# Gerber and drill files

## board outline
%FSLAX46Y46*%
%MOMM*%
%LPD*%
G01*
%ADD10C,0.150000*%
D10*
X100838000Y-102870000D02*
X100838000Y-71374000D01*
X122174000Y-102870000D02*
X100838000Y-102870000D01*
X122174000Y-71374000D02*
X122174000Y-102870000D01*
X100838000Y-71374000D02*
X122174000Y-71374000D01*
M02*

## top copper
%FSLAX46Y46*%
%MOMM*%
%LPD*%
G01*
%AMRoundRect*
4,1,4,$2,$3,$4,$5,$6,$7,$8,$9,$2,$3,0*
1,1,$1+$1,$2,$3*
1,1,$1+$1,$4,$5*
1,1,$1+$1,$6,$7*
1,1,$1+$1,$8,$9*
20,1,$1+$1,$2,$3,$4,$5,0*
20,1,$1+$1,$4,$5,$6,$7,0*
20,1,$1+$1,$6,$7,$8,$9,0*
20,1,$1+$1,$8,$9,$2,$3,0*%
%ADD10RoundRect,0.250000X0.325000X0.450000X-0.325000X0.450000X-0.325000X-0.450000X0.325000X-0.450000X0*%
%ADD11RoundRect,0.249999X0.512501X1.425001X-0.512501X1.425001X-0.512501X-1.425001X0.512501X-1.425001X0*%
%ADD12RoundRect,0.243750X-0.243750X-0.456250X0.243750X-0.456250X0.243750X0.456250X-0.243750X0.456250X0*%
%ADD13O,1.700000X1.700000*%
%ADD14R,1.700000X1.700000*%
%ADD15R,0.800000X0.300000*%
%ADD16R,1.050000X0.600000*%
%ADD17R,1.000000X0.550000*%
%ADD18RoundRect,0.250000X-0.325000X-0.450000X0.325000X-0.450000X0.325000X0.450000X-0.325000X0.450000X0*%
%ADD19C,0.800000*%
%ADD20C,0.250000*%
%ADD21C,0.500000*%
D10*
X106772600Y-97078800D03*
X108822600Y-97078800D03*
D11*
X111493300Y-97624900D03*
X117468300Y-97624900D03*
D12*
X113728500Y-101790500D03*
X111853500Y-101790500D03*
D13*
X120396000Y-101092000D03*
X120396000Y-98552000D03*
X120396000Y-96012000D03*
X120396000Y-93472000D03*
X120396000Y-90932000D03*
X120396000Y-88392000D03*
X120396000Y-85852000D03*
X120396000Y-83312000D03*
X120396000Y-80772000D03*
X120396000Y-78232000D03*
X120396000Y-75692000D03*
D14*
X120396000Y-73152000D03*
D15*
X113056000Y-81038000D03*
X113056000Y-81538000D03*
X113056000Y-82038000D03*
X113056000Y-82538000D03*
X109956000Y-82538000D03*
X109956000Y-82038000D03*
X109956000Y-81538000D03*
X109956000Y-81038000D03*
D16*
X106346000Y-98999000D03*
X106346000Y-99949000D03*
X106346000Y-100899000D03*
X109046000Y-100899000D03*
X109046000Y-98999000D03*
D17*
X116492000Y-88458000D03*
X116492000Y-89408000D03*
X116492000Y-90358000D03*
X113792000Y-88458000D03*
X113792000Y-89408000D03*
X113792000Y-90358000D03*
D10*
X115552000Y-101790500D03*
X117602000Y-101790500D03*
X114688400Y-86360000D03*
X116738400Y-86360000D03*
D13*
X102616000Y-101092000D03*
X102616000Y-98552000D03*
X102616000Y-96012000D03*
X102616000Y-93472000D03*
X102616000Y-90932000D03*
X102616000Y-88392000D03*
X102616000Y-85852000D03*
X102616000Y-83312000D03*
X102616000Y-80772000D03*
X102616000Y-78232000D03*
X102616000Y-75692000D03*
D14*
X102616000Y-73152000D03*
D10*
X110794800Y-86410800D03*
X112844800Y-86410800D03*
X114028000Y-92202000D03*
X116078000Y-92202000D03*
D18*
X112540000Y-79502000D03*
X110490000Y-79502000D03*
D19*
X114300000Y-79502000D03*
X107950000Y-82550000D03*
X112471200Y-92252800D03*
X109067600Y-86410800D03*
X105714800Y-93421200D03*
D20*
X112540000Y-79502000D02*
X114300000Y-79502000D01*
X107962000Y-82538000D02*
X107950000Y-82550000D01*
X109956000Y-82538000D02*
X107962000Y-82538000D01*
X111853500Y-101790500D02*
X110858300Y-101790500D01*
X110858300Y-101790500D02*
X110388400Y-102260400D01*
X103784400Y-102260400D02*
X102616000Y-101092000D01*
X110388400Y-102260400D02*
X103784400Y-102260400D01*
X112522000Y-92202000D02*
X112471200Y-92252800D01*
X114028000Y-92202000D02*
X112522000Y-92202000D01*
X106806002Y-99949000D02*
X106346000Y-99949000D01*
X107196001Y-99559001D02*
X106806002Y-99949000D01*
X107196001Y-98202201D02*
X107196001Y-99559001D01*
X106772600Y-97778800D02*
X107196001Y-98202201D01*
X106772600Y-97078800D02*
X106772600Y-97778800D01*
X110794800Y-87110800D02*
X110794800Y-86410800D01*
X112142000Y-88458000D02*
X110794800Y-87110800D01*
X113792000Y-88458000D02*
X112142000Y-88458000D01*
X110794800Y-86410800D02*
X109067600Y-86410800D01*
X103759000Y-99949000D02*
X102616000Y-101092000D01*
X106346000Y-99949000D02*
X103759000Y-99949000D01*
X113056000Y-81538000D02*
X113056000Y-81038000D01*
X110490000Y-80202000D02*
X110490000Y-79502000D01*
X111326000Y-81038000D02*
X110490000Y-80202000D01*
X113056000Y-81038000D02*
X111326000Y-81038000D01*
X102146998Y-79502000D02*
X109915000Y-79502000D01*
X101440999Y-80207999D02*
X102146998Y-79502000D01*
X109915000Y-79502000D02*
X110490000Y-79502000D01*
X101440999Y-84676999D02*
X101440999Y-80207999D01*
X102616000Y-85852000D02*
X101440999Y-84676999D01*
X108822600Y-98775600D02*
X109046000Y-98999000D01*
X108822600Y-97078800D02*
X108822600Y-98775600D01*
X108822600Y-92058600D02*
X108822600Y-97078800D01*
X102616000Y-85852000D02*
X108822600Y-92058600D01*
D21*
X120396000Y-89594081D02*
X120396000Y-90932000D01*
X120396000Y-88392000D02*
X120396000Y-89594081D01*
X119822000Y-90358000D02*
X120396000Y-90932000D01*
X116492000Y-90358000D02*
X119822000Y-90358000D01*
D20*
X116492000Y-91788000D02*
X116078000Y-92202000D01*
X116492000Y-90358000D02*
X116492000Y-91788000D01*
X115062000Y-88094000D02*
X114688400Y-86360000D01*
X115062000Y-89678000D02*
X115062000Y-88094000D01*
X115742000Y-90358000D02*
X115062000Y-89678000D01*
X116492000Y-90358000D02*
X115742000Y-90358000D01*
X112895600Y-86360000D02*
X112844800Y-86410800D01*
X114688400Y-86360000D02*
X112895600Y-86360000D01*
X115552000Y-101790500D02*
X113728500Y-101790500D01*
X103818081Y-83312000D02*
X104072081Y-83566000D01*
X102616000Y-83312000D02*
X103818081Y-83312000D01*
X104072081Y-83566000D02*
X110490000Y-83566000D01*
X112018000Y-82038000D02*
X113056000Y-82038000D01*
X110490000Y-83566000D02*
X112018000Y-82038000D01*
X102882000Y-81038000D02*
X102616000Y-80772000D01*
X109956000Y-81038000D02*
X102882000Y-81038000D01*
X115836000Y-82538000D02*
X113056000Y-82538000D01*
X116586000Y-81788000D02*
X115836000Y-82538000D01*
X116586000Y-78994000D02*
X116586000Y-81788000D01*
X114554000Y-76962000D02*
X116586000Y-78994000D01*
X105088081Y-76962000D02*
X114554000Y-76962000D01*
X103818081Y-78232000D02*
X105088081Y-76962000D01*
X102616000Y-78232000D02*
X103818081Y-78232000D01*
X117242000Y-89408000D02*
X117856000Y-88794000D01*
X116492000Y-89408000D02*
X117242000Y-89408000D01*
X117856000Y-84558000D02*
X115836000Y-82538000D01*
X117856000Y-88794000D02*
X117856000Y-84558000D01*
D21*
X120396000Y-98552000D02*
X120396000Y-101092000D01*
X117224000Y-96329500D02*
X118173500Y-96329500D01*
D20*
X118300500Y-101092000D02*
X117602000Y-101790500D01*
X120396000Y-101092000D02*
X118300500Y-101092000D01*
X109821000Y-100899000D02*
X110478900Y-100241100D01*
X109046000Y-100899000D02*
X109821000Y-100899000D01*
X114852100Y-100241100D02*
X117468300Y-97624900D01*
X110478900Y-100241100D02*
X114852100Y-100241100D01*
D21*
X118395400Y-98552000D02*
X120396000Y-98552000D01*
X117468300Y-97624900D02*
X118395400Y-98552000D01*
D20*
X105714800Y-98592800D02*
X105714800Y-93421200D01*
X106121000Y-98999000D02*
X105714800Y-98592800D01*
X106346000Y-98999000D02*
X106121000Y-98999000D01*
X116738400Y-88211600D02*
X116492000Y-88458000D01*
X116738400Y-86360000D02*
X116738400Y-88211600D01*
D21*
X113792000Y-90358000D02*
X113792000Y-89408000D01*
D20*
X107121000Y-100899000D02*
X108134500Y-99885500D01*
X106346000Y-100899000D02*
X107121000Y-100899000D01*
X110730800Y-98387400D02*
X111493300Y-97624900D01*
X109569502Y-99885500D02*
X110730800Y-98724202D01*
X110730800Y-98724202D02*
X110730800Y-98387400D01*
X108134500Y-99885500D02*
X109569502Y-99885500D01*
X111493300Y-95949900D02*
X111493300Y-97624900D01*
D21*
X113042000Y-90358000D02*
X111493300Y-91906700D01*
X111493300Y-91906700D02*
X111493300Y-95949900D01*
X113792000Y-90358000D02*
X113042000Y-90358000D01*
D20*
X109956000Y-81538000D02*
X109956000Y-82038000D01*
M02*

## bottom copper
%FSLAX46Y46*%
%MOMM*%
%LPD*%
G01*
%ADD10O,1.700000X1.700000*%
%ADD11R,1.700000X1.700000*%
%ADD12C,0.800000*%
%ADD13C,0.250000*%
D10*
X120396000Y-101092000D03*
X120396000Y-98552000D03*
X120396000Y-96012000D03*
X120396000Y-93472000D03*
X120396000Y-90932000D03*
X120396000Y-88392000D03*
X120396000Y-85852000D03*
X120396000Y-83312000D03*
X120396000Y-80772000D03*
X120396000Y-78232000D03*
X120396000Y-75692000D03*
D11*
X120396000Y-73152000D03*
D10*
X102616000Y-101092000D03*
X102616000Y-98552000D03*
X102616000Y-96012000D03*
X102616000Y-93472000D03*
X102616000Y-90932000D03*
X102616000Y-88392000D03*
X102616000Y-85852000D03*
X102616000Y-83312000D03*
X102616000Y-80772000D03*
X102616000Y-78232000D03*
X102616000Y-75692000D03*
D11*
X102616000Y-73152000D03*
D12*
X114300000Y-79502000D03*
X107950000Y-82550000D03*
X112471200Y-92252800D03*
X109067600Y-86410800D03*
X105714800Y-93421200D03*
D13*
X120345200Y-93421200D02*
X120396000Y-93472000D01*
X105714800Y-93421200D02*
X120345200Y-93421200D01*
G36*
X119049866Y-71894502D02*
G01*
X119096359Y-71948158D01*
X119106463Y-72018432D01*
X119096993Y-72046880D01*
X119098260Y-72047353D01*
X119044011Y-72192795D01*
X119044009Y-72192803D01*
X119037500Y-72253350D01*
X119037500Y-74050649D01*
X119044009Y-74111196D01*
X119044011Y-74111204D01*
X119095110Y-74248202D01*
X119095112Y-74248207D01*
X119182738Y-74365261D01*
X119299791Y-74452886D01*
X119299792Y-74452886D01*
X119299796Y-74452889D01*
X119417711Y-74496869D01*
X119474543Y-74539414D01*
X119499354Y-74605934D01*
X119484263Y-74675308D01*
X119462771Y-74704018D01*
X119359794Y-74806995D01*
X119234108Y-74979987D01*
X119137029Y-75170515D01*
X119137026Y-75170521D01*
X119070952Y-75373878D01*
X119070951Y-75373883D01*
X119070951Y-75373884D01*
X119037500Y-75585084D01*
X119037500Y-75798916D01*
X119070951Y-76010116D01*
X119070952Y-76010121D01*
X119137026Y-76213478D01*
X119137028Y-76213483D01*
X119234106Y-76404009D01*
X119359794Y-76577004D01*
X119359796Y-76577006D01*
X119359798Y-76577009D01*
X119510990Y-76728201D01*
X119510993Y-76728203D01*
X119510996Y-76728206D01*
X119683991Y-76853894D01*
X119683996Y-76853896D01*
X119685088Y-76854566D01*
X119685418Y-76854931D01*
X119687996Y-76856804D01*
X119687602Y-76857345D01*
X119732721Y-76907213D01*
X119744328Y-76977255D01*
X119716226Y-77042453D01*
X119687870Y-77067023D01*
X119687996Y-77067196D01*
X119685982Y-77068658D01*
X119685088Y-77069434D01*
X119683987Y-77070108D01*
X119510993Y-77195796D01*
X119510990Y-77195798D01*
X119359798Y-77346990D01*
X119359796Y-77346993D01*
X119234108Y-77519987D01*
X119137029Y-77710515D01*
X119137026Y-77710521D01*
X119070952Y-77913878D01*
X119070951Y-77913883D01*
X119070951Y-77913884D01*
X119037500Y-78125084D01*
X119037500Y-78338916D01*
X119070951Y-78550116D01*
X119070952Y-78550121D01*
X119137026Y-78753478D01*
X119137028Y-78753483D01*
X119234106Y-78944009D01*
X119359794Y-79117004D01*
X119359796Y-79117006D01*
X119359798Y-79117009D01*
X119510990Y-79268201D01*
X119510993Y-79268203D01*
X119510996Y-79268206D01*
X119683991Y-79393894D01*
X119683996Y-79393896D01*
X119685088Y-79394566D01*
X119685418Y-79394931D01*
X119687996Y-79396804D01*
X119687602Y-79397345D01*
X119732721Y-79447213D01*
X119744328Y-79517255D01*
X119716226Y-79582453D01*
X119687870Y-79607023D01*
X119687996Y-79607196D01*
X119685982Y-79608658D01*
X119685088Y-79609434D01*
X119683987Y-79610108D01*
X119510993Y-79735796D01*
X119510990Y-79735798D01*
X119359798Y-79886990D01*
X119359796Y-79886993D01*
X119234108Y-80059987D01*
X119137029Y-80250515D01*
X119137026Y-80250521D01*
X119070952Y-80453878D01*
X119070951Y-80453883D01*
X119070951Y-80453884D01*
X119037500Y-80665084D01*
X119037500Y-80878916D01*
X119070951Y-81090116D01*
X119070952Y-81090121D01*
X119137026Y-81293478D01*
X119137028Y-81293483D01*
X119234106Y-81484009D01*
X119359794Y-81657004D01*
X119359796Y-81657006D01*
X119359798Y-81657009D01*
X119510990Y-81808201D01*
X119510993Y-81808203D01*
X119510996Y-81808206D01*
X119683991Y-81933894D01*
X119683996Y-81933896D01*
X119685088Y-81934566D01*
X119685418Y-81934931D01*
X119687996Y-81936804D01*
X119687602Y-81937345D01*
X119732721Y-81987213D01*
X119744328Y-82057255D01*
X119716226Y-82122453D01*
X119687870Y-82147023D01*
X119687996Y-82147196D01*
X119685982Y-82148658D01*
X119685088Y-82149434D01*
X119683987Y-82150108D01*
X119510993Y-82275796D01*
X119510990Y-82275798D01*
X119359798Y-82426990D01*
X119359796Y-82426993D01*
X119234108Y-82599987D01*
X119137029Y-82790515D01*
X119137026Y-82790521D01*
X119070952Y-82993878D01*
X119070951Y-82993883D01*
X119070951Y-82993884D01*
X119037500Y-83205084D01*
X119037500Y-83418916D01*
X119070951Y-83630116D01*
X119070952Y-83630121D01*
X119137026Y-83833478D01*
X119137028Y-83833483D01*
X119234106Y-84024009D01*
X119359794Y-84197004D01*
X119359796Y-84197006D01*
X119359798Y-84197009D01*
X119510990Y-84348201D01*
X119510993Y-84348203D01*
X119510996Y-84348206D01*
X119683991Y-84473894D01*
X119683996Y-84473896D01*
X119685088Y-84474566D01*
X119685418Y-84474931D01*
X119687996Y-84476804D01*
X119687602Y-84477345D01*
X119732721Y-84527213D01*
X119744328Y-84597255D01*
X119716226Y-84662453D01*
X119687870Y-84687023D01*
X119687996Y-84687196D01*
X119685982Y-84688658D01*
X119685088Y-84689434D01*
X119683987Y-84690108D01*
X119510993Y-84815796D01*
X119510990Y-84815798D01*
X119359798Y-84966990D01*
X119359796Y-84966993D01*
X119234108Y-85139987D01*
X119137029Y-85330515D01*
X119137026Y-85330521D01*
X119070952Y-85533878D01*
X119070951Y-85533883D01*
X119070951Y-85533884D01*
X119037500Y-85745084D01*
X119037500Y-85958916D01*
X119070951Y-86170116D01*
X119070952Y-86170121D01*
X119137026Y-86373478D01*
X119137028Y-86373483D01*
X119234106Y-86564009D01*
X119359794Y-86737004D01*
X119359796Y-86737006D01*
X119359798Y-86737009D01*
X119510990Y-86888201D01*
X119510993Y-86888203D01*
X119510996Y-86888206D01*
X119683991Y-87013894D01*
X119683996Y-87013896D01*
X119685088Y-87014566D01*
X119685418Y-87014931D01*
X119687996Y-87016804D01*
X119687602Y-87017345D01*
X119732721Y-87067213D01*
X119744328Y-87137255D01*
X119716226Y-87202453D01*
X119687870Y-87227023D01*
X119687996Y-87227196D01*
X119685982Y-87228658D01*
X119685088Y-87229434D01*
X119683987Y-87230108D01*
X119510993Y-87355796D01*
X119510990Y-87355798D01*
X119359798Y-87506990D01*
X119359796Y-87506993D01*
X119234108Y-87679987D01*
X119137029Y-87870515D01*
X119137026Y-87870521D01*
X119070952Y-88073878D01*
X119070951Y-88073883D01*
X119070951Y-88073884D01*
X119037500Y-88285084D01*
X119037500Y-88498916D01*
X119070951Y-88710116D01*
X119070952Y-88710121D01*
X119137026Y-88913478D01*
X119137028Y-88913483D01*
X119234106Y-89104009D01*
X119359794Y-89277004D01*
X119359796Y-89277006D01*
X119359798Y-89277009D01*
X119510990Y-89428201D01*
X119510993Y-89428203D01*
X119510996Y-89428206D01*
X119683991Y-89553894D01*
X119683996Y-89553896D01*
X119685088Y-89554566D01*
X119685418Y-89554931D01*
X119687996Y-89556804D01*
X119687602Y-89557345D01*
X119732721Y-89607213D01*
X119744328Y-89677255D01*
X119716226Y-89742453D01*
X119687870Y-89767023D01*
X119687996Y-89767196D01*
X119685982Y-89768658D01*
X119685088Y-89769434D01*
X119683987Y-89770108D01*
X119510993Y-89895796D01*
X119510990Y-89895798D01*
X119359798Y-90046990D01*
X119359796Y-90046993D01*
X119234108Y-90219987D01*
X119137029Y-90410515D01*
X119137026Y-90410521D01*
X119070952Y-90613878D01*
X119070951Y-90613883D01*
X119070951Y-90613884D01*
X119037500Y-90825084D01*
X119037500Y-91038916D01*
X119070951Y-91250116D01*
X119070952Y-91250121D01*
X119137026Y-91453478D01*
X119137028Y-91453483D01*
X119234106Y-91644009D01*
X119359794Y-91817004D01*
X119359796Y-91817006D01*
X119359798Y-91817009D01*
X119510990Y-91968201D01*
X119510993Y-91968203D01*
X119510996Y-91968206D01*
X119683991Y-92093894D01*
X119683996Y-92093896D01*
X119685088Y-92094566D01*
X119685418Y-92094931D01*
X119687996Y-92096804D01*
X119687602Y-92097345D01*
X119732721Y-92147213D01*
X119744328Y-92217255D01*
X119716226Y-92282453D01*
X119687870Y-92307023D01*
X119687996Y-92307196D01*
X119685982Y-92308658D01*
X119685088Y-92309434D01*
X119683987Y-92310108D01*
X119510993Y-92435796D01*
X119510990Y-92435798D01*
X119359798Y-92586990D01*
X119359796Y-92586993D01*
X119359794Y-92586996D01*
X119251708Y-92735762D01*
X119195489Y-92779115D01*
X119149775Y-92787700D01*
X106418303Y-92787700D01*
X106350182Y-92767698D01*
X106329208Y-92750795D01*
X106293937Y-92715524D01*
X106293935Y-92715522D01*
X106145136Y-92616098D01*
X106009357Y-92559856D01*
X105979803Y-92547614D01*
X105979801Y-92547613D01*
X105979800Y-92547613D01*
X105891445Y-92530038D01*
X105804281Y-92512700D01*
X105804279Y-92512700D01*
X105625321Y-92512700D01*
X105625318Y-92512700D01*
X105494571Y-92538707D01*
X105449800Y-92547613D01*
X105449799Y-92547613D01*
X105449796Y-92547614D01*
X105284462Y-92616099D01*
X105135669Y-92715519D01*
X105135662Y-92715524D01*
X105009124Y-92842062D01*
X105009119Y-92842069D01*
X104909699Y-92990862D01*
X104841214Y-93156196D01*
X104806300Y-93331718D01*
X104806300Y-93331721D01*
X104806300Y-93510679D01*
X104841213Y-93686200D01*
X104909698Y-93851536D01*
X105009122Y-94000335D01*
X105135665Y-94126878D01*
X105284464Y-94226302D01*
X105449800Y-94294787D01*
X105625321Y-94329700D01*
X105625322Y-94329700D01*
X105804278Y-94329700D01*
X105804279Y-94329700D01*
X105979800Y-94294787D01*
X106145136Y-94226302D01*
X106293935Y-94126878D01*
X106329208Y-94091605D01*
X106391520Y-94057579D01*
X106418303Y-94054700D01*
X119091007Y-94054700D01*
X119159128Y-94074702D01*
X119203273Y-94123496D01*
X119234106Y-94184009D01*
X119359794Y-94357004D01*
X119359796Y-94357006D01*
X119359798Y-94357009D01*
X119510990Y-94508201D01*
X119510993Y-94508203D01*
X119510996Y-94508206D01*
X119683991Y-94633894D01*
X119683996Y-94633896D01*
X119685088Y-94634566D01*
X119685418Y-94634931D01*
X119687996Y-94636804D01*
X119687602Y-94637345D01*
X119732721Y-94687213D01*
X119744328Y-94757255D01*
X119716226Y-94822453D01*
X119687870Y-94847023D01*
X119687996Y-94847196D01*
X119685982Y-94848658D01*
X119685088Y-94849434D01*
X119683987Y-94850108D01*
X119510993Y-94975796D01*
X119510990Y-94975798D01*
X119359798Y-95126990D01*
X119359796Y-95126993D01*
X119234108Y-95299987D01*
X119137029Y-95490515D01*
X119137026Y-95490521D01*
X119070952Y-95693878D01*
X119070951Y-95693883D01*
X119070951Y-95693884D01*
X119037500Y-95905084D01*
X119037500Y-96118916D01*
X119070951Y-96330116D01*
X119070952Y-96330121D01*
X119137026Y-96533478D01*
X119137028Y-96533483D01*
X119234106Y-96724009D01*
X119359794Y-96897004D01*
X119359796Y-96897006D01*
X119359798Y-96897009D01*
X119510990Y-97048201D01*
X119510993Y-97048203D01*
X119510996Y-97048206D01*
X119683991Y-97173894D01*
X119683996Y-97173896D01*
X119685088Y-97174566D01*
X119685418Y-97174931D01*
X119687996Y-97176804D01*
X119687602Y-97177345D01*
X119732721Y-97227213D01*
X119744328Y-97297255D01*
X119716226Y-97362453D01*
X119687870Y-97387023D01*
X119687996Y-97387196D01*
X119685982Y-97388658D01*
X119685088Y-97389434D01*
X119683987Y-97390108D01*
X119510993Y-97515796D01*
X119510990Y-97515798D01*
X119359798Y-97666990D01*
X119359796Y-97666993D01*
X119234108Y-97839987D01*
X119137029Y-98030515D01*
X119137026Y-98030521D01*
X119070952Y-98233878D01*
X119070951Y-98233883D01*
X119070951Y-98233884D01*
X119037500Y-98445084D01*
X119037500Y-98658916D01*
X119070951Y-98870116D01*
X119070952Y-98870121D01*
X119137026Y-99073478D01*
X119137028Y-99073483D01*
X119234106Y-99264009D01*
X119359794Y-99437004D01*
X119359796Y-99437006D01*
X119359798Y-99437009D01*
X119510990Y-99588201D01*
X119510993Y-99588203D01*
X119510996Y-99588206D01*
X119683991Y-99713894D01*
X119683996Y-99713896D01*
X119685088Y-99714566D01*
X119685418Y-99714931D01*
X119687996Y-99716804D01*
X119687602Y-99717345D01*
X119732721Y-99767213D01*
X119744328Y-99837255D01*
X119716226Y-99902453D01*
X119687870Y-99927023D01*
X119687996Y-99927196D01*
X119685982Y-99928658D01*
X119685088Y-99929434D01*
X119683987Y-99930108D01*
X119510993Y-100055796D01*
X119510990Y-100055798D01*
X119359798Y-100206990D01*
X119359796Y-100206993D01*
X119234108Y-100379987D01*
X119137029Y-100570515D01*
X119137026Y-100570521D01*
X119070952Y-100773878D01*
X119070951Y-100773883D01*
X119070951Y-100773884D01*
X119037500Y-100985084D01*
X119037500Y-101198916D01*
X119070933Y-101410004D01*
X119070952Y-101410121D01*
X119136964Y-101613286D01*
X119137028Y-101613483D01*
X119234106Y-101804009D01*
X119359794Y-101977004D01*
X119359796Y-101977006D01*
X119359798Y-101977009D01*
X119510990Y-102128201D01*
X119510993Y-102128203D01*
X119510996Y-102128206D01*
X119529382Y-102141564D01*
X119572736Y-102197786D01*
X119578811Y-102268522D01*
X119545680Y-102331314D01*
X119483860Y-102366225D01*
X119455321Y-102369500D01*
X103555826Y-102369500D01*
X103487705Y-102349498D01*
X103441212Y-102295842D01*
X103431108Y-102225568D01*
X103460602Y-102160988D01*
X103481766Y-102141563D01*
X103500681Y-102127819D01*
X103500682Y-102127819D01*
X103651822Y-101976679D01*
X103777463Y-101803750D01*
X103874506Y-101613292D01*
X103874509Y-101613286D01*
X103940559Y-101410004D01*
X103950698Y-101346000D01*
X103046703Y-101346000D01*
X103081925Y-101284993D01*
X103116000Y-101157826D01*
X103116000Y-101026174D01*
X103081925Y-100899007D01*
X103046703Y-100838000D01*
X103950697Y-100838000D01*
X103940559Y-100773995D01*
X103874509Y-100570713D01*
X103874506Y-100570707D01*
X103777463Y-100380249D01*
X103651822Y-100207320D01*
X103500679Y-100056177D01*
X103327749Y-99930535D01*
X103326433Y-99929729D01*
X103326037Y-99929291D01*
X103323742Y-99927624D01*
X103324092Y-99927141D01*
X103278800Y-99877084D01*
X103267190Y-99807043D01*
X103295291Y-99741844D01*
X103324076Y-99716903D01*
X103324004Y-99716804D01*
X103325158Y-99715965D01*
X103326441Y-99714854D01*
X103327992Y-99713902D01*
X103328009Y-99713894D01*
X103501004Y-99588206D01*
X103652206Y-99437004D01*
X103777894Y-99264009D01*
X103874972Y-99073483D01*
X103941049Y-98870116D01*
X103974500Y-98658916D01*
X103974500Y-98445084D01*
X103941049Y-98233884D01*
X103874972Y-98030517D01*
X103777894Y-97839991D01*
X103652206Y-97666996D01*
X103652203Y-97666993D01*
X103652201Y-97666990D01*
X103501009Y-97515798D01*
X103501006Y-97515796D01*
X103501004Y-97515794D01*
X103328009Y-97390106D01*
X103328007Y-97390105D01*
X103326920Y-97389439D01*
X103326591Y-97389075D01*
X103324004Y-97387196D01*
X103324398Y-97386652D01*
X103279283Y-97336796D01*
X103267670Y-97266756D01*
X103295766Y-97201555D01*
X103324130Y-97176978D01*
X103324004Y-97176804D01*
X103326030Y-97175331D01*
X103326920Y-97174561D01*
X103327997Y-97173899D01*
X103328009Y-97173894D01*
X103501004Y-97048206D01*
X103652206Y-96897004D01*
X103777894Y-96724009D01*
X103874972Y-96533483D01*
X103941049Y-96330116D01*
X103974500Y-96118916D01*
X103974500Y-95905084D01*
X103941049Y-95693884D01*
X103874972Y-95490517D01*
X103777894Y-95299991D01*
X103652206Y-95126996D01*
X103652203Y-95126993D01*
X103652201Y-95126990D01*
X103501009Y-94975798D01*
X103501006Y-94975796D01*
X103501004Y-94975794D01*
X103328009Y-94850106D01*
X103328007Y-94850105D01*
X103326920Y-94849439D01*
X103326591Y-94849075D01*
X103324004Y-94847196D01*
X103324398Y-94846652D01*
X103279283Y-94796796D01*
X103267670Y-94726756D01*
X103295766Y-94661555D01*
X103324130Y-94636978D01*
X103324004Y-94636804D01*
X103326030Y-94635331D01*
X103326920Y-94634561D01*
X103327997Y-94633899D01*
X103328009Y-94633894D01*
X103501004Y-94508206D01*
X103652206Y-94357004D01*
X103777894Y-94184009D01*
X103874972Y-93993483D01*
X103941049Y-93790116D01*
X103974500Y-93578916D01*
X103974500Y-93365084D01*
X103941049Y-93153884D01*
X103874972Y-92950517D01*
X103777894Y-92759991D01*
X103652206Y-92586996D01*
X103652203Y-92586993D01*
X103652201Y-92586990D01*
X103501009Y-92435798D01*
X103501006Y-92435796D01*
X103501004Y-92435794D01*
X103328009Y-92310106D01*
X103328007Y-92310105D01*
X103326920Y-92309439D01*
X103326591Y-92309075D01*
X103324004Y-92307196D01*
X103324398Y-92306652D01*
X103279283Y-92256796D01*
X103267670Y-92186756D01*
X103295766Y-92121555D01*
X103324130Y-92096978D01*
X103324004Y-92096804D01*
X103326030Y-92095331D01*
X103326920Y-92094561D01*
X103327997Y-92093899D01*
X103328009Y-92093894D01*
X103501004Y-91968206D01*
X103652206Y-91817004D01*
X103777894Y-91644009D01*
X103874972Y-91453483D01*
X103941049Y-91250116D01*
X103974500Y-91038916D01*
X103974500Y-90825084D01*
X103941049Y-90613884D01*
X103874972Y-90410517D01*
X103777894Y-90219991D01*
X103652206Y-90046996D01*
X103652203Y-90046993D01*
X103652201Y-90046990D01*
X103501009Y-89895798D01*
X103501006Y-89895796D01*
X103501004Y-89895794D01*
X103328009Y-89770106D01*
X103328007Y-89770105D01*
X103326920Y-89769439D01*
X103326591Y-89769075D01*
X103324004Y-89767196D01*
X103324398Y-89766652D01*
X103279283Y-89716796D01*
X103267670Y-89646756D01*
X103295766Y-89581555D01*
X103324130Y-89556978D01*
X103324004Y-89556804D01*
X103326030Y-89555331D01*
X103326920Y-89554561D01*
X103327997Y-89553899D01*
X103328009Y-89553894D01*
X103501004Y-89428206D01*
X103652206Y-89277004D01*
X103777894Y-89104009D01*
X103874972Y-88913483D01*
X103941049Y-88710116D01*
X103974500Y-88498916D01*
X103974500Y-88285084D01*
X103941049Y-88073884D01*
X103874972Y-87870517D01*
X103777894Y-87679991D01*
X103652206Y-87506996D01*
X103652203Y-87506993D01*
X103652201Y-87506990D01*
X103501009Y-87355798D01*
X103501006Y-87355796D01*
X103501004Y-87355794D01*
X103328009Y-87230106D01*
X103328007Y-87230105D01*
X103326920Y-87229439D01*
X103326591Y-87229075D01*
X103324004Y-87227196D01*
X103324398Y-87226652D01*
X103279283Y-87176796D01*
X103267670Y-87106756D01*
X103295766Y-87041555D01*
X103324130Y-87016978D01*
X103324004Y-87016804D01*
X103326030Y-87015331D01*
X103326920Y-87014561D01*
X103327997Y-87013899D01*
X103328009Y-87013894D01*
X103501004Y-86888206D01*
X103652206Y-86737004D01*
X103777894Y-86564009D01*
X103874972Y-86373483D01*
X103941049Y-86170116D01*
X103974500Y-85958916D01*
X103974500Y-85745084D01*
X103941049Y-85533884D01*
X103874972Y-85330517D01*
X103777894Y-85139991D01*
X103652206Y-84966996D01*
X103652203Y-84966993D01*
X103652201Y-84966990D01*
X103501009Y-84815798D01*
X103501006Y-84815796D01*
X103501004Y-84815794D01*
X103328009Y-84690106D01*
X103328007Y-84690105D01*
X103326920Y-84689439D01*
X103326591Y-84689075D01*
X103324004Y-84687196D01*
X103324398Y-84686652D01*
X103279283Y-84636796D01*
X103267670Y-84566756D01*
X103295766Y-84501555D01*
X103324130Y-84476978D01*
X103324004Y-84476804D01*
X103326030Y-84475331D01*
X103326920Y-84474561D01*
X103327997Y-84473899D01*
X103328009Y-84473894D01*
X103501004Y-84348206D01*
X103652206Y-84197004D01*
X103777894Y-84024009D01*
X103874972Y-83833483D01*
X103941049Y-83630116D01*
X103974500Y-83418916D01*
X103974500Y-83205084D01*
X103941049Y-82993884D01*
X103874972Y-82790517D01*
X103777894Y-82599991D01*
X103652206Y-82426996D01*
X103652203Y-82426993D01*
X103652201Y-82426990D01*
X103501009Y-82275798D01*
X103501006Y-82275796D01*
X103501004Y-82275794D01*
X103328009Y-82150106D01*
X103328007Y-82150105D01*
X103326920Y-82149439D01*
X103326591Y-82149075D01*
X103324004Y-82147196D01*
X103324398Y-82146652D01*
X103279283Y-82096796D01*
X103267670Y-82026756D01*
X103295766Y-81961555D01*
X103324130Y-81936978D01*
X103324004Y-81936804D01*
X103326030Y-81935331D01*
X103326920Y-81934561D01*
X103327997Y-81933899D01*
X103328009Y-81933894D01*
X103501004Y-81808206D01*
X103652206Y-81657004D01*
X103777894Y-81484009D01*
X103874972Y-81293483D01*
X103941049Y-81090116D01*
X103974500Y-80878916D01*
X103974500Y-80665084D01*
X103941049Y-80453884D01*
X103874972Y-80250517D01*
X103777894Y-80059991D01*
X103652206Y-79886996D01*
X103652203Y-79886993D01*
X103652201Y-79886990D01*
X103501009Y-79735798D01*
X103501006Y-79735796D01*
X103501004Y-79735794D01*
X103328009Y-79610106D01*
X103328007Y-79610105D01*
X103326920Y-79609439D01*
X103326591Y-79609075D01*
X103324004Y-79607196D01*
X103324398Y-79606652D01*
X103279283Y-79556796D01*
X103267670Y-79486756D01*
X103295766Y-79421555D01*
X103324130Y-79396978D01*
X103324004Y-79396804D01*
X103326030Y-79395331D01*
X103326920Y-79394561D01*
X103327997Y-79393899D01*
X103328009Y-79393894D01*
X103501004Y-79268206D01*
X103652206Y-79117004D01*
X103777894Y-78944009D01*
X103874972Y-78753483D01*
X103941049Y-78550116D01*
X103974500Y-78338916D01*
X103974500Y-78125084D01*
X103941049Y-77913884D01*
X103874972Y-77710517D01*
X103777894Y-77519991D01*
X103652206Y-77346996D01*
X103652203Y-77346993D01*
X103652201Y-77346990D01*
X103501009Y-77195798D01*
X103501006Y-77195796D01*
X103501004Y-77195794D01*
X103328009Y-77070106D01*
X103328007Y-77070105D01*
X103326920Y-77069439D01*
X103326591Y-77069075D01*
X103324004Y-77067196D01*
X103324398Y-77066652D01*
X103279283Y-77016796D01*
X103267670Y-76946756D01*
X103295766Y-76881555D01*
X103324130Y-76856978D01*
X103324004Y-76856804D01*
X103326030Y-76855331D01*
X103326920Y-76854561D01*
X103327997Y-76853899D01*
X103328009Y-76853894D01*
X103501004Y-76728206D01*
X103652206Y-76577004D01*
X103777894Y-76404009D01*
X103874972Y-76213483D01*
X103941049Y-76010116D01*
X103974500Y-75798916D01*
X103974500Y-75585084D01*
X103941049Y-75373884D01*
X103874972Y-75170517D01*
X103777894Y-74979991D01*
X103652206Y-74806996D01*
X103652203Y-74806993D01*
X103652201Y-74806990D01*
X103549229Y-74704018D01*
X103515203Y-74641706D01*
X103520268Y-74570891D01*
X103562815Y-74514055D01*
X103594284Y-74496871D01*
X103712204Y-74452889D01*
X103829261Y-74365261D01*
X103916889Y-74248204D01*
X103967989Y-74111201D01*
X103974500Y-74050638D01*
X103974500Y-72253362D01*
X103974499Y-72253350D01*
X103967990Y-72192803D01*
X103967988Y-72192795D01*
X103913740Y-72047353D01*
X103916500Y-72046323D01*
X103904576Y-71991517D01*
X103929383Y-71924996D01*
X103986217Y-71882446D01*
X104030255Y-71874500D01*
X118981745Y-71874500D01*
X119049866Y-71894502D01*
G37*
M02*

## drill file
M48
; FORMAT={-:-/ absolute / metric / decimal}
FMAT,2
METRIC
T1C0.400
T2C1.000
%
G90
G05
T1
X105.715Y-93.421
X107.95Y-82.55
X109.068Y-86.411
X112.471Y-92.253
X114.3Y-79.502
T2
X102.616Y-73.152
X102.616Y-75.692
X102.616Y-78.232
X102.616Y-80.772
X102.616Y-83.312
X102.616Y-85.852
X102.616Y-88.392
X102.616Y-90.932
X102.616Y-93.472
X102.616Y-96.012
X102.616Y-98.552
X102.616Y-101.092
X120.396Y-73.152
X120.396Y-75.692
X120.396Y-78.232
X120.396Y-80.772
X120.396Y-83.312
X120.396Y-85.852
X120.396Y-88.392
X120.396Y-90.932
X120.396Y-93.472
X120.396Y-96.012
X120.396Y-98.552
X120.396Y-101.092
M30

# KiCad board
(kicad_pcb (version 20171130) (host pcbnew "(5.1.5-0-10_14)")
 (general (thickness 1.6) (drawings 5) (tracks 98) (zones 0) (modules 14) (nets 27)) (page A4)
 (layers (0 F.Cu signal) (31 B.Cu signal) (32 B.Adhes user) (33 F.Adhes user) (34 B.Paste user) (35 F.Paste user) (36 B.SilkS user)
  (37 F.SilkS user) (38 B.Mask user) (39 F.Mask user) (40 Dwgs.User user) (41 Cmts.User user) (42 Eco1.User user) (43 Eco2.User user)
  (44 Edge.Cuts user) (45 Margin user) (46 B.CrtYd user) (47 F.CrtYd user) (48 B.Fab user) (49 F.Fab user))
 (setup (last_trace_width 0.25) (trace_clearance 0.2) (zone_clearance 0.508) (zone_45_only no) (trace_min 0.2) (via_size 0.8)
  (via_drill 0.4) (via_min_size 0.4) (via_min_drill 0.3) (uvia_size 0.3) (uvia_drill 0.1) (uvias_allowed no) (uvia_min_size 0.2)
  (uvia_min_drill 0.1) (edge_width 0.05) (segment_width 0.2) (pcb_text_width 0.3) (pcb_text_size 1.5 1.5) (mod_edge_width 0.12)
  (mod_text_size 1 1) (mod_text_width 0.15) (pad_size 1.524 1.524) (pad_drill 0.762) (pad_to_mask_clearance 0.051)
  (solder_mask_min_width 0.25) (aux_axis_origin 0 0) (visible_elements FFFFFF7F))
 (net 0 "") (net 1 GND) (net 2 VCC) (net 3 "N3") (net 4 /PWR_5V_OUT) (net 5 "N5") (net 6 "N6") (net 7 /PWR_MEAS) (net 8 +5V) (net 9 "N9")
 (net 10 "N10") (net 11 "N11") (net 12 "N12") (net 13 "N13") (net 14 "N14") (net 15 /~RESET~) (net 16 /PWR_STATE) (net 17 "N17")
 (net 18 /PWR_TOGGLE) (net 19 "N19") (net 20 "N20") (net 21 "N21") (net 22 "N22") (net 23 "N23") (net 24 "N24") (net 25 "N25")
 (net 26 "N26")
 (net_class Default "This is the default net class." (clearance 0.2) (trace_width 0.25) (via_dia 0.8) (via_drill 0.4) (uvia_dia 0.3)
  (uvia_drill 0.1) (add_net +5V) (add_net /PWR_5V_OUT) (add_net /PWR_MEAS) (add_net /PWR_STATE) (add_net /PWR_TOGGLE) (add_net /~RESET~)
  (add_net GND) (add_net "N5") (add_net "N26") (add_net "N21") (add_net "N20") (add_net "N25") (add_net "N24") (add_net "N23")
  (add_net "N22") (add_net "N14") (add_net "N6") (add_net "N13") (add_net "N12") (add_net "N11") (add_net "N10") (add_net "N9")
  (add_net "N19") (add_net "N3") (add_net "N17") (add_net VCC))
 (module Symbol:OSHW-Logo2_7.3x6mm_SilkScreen (layer B.Cu) (at 111.7981 77.3684)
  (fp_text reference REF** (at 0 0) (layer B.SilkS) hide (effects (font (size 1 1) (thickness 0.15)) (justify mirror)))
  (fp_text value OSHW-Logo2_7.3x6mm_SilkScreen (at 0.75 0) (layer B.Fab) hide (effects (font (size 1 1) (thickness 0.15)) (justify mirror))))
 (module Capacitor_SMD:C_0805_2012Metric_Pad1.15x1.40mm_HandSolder (layer F.Cu) (at 107.7976 97.0788 180)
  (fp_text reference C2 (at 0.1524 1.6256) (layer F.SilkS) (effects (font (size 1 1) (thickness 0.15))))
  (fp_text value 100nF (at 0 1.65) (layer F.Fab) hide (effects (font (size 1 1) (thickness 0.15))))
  (pad 2 smd roundrect (at 1.025 0 180) (size 1.15 1.4) (layers F.Cu F.Paste F.Mask) (roundrect_rratio 0.217391) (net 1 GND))
  (pad 1 smd roundrect (at -1.025 0 180) (size 1.15 1.4) (layers F.Cu F.Paste F.Mask) (roundrect_rratio 0.217391) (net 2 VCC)))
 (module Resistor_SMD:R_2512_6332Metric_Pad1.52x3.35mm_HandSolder (layer F.Cu) (at 114.4808 97.6249 180)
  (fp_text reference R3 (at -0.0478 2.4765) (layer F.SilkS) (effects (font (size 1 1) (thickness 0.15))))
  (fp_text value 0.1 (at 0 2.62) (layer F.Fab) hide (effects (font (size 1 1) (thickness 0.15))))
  (pad 2 smd roundrect (at 2.9875 0 180) (size 1.525 3.35) (layers F.Cu F.Paste F.Mask) (roundrect_rratio 0.163934) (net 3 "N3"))
  (pad 1 smd roundrect (at -2.9875 0 180) (size 1.525 3.35) (layers F.Cu F.Paste F.Mask) (roundrect_rratio 0.163934) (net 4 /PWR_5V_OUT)))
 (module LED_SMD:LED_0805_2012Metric (layer F.Cu) (at 112.791 101.7905)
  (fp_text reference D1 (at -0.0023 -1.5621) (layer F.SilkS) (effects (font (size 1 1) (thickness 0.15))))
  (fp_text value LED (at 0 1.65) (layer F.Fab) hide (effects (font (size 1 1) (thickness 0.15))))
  (pad 2 smd roundrect (at 0.9375 0) (size 0.975 1.4) (layers F.Cu F.Paste F.Mask) (roundrect_rratio 0.25) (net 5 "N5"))
  (pad 1 smd roundrect (at -0.9375 0) (size 0.975 1.4) (layers F.Cu F.Paste F.Mask) (roundrect_rratio 0.25) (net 1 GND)))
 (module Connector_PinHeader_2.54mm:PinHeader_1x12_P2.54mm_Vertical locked (layer B.Cu) (at 120.396 73.152 180)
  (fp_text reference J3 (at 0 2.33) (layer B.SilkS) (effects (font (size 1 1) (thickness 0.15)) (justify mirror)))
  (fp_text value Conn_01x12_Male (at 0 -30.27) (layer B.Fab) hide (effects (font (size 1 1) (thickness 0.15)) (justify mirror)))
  (pad 12 thru_hole oval (at 0 -27.94 180) (size 1.7 1.7) (drill 1) (layers *.Cu *.Mask) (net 4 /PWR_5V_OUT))
  (pad 11 thru_hole oval (at 0 -25.4 180) (size 1.7 1.7) (drill 1) (layers *.Cu *.Mask) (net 4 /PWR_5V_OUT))
  (pad 10 thru_hole oval (at 0 -22.86 180) (size 1.7 1.7) (drill 1) (layers *.Cu *.Mask) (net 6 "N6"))
  (pad 9 thru_hole oval (at 0 -20.32 180) (size 1.7 1.7) (drill 1) (layers *.Cu *.Mask) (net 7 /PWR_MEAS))
  (pad 8 thru_hole oval (at 0 -17.78 180) (size 1.7 1.7) (drill 1) (layers *.Cu *.Mask) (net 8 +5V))
  (pad 7 thru_hole oval (at 0 -15.24 180) (size 1.7 1.7) (drill 1) (layers *.Cu *.Mask) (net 8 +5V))
  (pad 6 thru_hole oval (at 0 -12.7 180) (size 1.7 1.7) (drill 1) (layers *.Cu *.Mask) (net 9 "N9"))
  (pad 5 thru_hole oval (at 0 -10.16 180) (size 1.7 1.7) (drill 1) (layers *.Cu *.Mask) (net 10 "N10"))
  (pad 4 thru_hole oval (at 0 -7.62 180) (size 1.7 1.7) (drill 1) (layers *.Cu *.Mask) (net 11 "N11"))
  (pad 3 thru_hole oval (at 0 -5.08 180) (size 1.7 1.7) (drill 1) (layers *.Cu *.Mask) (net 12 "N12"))
  (pad 2 thru_hole oval (at 0 -2.54 180) (size 1.7 1.7) (drill 1) (layers *.Cu *.Mask) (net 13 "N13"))
  (pad 1 thru_hole rect (at 0 0 180) (size 1.7 1.7) (drill 1) (layers *.Cu *.Mask) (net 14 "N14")))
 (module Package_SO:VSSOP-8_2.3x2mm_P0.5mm (layer F.Cu) (at 111.506 81.788)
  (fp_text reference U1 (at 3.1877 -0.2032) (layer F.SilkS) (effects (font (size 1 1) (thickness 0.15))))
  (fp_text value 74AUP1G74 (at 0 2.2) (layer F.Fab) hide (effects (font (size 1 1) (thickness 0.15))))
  (pad 8 smd rect (at 1.55 -0.75 270) (size 0.3 0.8) (layers F.Cu F.Paste F.Mask) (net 2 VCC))
  (pad 7 smd rect (at 1.55 -0.25 270) (size 0.3 0.8) (layers F.Cu F.Paste F.Mask) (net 2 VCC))
  (pad 6 smd rect (at 1.55 0.25 270) (size 0.3 0.8) (layers F.Cu F.Paste F.Mask) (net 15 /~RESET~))
  (pad 5 smd rect (at 1.55 0.75 270) (size 0.3 0.8) (layers F.Cu F.Paste F.Mask) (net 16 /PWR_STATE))
  (pad 4 smd rect (at -1.55 0.75 270) (size 0.3 0.8) (layers F.Cu F.Paste F.Mask) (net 1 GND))
  (pad 3 smd rect (at -1.55 0.25 270) (size 0.3 0.8) (layers F.Cu F.Paste F.Mask) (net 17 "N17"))
  (pad 2 smd rect (at -1.55 -0.25 270) (size 0.3 0.8) (layers F.Cu F.Paste F.Mask) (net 17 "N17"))
  (pad 1 smd rect (at -1.55 -0.75 270) (size 0.3 0.8) (layers F.Cu F.Paste F.Mask) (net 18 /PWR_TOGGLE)))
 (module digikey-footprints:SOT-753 (layer F.Cu) (at 107.696 99.949 270)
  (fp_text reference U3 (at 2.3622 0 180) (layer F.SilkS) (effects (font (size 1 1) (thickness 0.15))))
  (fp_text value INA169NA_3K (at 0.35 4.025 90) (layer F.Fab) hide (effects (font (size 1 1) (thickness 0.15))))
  (pad 1 smd rect (at -0.95 1.35 270) (size 0.6 1.05) (layers F.Cu F.Paste F.Mask) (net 7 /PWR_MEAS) (solder_mask_margin 0.07))
  (pad 2 smd rect (at 0 1.35 270) (size 0.6 1.05) (layers F.Cu F.Paste F.Mask) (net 1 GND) (solder_mask_margin 0.07))
  (pad 3 smd rect (at 0.95 1.35 270) (size 0.6 1.05) (layers F.Cu F.Paste F.Mask) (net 3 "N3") (solder_mask_margin 0.07))
  (pad 4 smd rect (at 0.95 -1.35 270) (size 0.6 1.05) (layers F.Cu F.Paste F.Mask) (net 4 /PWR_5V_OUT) (solder_mask_margin 0.07))
  (pad 5 smd rect (at -0.95 -1.35 270) (size 0.6 1.05) (layers F.Cu F.Paste F.Mask) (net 2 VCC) (solder_mask_margin 0.07)))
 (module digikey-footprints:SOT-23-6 (layer F.Cu) (at 115.142 89.408 270)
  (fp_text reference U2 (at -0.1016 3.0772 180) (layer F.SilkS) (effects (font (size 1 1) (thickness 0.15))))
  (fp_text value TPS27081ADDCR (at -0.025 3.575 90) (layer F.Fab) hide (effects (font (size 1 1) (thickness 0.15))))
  (pad 6 smd rect (at -0.95 -1.35 270) (size 0.55 1) (layers F.Cu F.Paste F.Mask) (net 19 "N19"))
  (pad 5 smd rect (at 0 -1.35 270) (size 0.55 1) (layers F.Cu F.Paste F.Mask) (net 16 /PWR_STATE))
  (pad 4 smd rect (at 0.95 -1.35 270) (size 0.55 1) (layers F.Cu F.Paste F.Mask) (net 8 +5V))
  (pad 1 smd rect (at -0.95 1.35 270) (size 0.55 1) (layers F.Cu F.Paste F.Mask) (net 1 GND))
  (pad 2 smd rect (at 0 1.35 270) (size 0.55 1) (layers F.Cu F.Paste F.Mask) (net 3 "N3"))
  (pad 3 smd rect (at 0.95 1.35 270) (size 0.55 1) (layers F.Cu F.Paste F.Mask) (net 3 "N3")))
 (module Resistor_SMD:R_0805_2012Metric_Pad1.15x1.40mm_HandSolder (layer F.Cu) (at 116.577 101.7905 180)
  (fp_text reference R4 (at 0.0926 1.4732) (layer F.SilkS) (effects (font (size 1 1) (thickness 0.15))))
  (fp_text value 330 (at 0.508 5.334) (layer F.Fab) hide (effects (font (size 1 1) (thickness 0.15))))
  (pad 2 smd roundrect (at 1.025 0 180) (size 1.15 1.4) (layers F.Cu F.Paste F.Mask) (roundrect_rratio 0.217391) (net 5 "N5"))
  (pad 1 smd roundrect (at -1.025 0 180) (size 1.15 1.4) (layers F.Cu F.Paste F.Mask) (roundrect_rratio 0.217391) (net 4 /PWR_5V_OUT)))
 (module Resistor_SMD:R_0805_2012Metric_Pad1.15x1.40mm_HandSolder (layer F.Cu) (at 115.7134 86.36 180)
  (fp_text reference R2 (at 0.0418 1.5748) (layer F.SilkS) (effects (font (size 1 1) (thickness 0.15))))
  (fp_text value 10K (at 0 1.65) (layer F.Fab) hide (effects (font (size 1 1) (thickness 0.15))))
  (pad 2 smd roundrect (at 1.025 0 180) (size 1.15 1.4) (layers F.Cu F.Paste F.Mask) (roundrect_rratio 0.217391) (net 8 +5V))
  (pad 1 smd roundrect (at -1.025 0 180) (size 1.15 1.4) (layers F.Cu F.Paste F.Mask) (roundrect_rratio 0.217391) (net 19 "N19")))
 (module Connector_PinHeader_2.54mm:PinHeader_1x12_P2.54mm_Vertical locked (layer B.Cu) (at 102.616 73.152 180)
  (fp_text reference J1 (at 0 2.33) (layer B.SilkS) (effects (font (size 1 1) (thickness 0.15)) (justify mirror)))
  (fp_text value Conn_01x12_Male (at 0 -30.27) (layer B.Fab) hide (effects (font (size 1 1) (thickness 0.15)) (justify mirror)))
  (pad 12 thru_hole oval (at 0 -27.94 180) (size 1.7 1.7) (drill 1) (layers *.Cu *.Mask) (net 1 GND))
  (pad 11 thru_hole oval (at 0 -25.4 180) (size 1.7 1.7) (drill 1) (layers *.Cu *.Mask) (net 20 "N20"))
  (pad 10 thru_hole oval (at 0 -22.86 180) (size 1.7 1.7) (drill 1) (layers *.Cu *.Mask) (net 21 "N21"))
  (pad 9 thru_hole oval (at 0 -20.32 180) (size 1.7 1.7) (drill 1) (layers *.Cu *.Mask) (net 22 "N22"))
  (pad 8 thru_hole oval (at 0 -17.78 180) (size 1.7 1.7) (drill 1) (layers *.Cu *.Mask) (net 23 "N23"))
  (pad 7 thru_hole oval (at 0 -15.24 180) (size 1.7 1.7) (drill 1) (layers *.Cu *.Mask) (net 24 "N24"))
  (pad 6 thru_hole oval (at 0 -12.7 180) (size 1.7 1.7) (drill 1) (layers *.Cu *.Mask) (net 2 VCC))
  (pad 5 thru_hole oval (at 0 -10.16 180) (size 1.7 1.7) (drill 1) (layers *.Cu *.Mask) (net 15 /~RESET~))
  (pad 4 thru_hole oval (at 0 -7.62 180) (size 1.7 1.7) (drill 1) (layers *.Cu *.Mask) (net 18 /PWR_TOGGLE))
  (pad 3 thru_hole oval (at 0 -5.08 180) (size 1.7 1.7) (drill 1) (layers *.Cu *.Mask) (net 16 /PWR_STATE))
  (pad 2 thru_hole oval (at 0 -2.54 180) (size 1.7 1.7) (drill 1) (layers *.Cu *.Mask) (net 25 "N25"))
  (pad 1 thru_hole rect (at 0 0 180) (size 1.7 1.7) (drill 1) (layers *.Cu *.Mask) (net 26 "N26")))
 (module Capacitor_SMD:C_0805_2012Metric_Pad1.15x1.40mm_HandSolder (layer F.Cu) (at 111.8198 86.4108 180)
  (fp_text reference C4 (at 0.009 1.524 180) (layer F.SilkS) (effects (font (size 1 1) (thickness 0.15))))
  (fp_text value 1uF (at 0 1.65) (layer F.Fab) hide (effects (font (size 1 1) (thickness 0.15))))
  (pad 2 smd roundrect (at 1.025 0 180) (size 1.15 1.4) (layers F.Cu F.Paste F.Mask) (roundrect_rratio 0.217391) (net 1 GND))
  (pad 1 smd roundrect (at -1.025 0 180) (size 1.15 1.4) (layers F.Cu F.Paste F.Mask) (roundrect_rratio 0.217391) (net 8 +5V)))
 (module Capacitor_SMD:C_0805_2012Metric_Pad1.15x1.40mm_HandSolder (layer F.Cu) (at 115.053 92.202 180)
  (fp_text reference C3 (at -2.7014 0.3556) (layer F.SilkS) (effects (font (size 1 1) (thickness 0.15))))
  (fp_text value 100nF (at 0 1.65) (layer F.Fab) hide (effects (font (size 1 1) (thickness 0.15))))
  (pad 2 smd roundrect (at 1.025 0 180) (size 1.15 1.4) (layers F.Cu F.Paste F.Mask) (roundrect_rratio 0.217391) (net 1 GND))
  (pad 1 smd roundrect (at -1.025 0 180) (size 1.15 1.4) (layers F.Cu F.Paste F.Mask) (roundrect_rratio 0.217391) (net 8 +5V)))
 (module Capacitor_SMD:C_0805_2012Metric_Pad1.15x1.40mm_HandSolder (layer F.Cu) (at 111.515 79.502)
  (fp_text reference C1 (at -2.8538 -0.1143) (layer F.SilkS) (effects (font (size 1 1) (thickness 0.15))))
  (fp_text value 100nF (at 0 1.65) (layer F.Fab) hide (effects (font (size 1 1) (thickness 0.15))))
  (pad 2 smd roundrect (at 1.025 0) (size 1.15 1.4) (layers F.Cu F.Paste F.Mask) (roundrect_rratio 0.217391) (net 1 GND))
  (pad 1 smd roundrect (at -1.025 0) (size 1.15 1.4) (layers F.Cu F.Paste F.Mask) (roundrect_rratio 0.217391) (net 2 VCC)))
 (gr_line (start 100.838 102.87) (end 100.838 71.374) (layer Edge.Cuts) (width 0.15))
 (gr_line (start 122.174 102.87) (end 100.838 102.87) (layer Edge.Cuts) (width 0.15))
 (gr_line (start 122.174 71.374) (end 122.174 102.87) (layer Edge.Cuts) (width 0.15))
 (gr_line (start 100.838 71.374) (end 122.174 71.374) (layer Edge.Cuts) (width 0.15))
 (via (at 114.3 79.502) (size 0.8) (drill 0.4) (layers F.Cu B.Cu) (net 1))
 (segment (start 112.54 79.502) (end 114.3 79.502) (width 0.25) (layer F.Cu) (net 1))
 (via (at 107.95 82.55) (size 0.8) (drill 0.4) (layers F.Cu B.Cu) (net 1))
 (segment (start 107.962 82.538) (end 107.95 82.55) (width 0.25) (layer F.Cu) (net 1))
 (segment (start 109.956 82.538) (end 107.962 82.538) (width 0.25) (layer F.Cu) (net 1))
 (segment (start 111.8535 101.7905) (end 110.8583 101.7905) (width 0.25) (layer F.Cu) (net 1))
 (segment (start 110.8583 101.7905) (end 110.3884 102.2604) (width 0.25) (layer F.Cu) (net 1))
 (segment (start 103.7844 102.2604) (end 102.616 101.092) (width 0.25) (layer F.Cu) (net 1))
 (segment (start 110.3884 102.2604) (end 103.7844 102.2604) (width 0.25) (layer F.Cu) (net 1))
 (via (at 112.4712 92.2528) (size 0.8) (drill 0.4) (layers F.Cu B.Cu) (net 1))
 (segment (start 112.522 92.202) (end 112.4712 92.2528) (width 0.25) (layer F.Cu) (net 1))
 (segment (start 114.028 92.202) (end 112.522 92.202) (width 0.25) (layer F.Cu) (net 1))
 (segment (start 106.806002 99.949) (end 106.346 99.949) (width 0.25) (layer F.Cu) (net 1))
 (segment (start 107.196001 99.559001) (end 106.806002 99.949) (width 0.25) (layer F.Cu) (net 1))
 (segment (start 107.196001 98.202201) (end 107.196001 99.559001) (width 0.25) (layer F.Cu) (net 1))
 (segment (start 106.7726 97.7788) (end 107.196001 98.202201) (width 0.25) (layer F.Cu) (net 1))
 (segment (start 106.7726 97.0788) (end 106.7726 97.7788) (width 0.25) (layer F.Cu) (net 1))
 (segment (start 110.7948 87.1108) (end 110.7948 86.4108) (width 0.25) (layer F.Cu) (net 1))
 (segment (start 112.142 88.458) (end 110.7948 87.1108) (width 0.25) (layer F.Cu) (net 1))
 (segment (start 113.792 88.458) (end 112.142 88.458) (width 0.25) (layer F.Cu) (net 1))
 (via (at 109.0676 86.4108) (size 0.8) (drill 0.4) (layers F.Cu B.Cu) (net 1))
 (segment (start 110.7948 86.4108) (end 109.0676 86.4108) (width 0.25) (layer F.Cu) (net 1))
 (segment (start 103.759 99.949) (end 102.616 101.092) (width 0.25) (layer F.Cu) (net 1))
 (segment (start 106.346 99.949) (end 103.759 99.949) (width 0.25) (layer F.Cu) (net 1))
 (segment (start 113.056 81.538) (end 113.056 81.038) (width 0.25) (layer F.Cu) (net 2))
 (segment (start 110.49 80.202) (end 110.49 79.502) (width 0.25) (layer F.Cu) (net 2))
 (segment (start 111.326 81.038) (end 110.49 80.202) (width 0.25) (layer F.Cu) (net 2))
 (segment (start 113.056 81.038) (end 111.326 81.038) (width 0.25) (layer F.Cu) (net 2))
 (segment (start 102.146998 79.502) (end 109.915 79.502) (width 0.25) (layer F.Cu) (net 2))
 (segment (start 101.440999 80.207999) (end 102.146998 79.502) (width 0.25) (layer F.Cu) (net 2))
 (segment (start 109.915 79.502) (end 110.49 79.502) (width 0.25) (layer F.Cu) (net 2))
 (segment (start 101.440999 84.676999) (end 101.440999 80.207999) (width 0.25) (layer F.Cu) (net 2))
 (segment (start 102.616 85.852) (end 101.440999 84.676999) (width 0.25) (layer F.Cu) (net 2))
 (segment (start 108.8226 98.7756) (end 109.046 98.999) (width 0.25) (layer F.Cu) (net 2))
 (segment (start 108.8226 97.0788) (end 108.8226 98.7756) (width 0.25) (layer F.Cu) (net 2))
 (segment (start 108.8226 92.0586) (end 108.8226 97.0788) (width 0.25) (layer F.Cu) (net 2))
 (segment (start 102.616 85.852) (end 108.8226 92.0586) (width 0.25) (layer F.Cu) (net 2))
 (segment (start 120.396 89.594081) (end 120.396 90.932) (width 0.5) (layer F.Cu) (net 8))
 (segment (start 120.396 88.392) (end 120.396 89.594081) (width 0.5) (layer F.Cu) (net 8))
 (segment (start 119.822 90.358) (end 120.396 90.932) (width 0.5) (layer F.Cu) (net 8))
 (segment (start 116.492 90.358) (end 119.822 90.358) (width 0.5) (layer F.Cu) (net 8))
 (segment (start 116.492 91.788) (end 116.078 92.202) (width 0.25) (layer F.Cu) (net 8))
 (segment (start 116.492 90.358) (end 116.492 91.788) (width 0.25) (layer F.Cu) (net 8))
 (segment (start 115.062 88.094) (end 114.6884 86.36) (width 0.25) (layer F.Cu) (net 8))
 (segment (start 115.062 89.678) (end 115.062 88.094) (width 0.25) (layer F.Cu) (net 8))
 (segment (start 115.742 90.358) (end 115.062 89.678) (width 0.25) (layer F.Cu) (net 8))
 (segment (start 116.492 90.358) (end 115.742 90.358) (width 0.25) (layer F.Cu) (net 8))
 (segment (start 112.8956 86.36) (end 112.8448 86.4108) (width 0.25) (layer F.Cu) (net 8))
 (segment (start 114.6884 86.36) (end 112.8956 86.36) (width 0.25) (layer F.Cu) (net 8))
 (segment (start 115.552 101.7905) (end 113.7285 101.7905) (width 0.25) (layer F.Cu) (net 5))
 (segment (start 103.818081 83.312) (end 104.072081 83.566) (width 0.25) (layer F.Cu) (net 15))
 (segment (start 102.616 83.312) (end 103.818081 83.312) (width 0.25) (layer F.Cu) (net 15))
 (segment (start 104.072081 83.566) (end 110.49 83.566) (width 0.25) (layer F.Cu) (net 15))
 (segment (start 112.018 82.038) (end 113.056 82.038) (width 0.25) (layer F.Cu) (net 15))
 (segment (start 110.49 83.566) (end 112.018 82.038) (width 0.25) (layer F.Cu) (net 15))
 (segment (start 102.882 81.038) (end 102.616 80.772) (width 0.25) (layer F.Cu) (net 18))
 (segment (start 109.956 81.038) (end 102.882 81.038) (width 0.25) (layer F.Cu) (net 18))
 (segment (start 115.836 82.538) (end 113.056 82.538) (width 0.25) (layer F.Cu) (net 16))
 (segment (start 116.586 81.788) (end 115.836 82.538) (width 0.25) (layer F.Cu) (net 16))
 (segment (start 116.586 78.994) (end 116.586 81.788) (width 0.25) (layer F.Cu) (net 16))
 (segment (start 114.554 76.962) (end 116.586 78.994) (width 0.25) (layer F.Cu) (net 16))
 (segment (start 105.088081 76.962) (end 114.554 76.962) (width 0.25) (layer F.Cu) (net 16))
 (segment (start 103.818081 78.232) (end 105.088081 76.962) (width 0.25) (layer F.Cu) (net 16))
 (segment (start 102.616 78.232) (end 103.818081 78.232) (width 0.25) (layer F.Cu) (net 16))
 (segment (start 117.242 89.408) (end 117.856 88.794) (width 0.25) (layer F.Cu) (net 16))
 (segment (start 116.492 89.408) (end 117.242 89.408) (width 0.25) (layer F.Cu) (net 16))
 (segment (start 117.856 84.558) (end 115.836 82.538) (width 0.25) (layer F.Cu) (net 16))
 (segment (start 117.856 88.794) (end 117.856 84.558) (width 0.25) (layer F.Cu) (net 16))
 (segment (start 120.396 98.552) (end 120.396 101.092) (width 0.5) (layer F.Cu) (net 4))
 (segment (start 117.224 96.3295) (end 118.1735 96.3295) (width 0.5) (layer F.Cu) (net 4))
 (segment (start 118.3005 101.092) (end 117.602 101.7905) (width 0.25) (layer F.Cu) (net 4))
 (segment (start 120.396 101.092) (end 118.3005 101.092) (width 0.25) (layer F.Cu) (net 4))
 (segment (start 109.821 100.899) (end 110.4789 100.2411) (width 0.25) (layer F.Cu) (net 4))
 (segment (start 109.046 100.899) (end 109.821 100.899) (width 0.25) (layer F.Cu) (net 4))
 (segment (start 114.8521 100.2411) (end 117.4683 97.6249) (width 0.25) (layer F.Cu) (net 4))
 (segment (start 110.4789 100.2411) (end 114.8521 100.2411) (width 0.25) (layer F.Cu) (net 4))
 (segment (start 118.3954 98.552) (end 120.396 98.552) (width 0.5) (layer F.Cu) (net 4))
 (segment (start 117.4683 97.6249) (end 118.3954 98.552) (width 0.5) (layer F.Cu) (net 4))
 (via (at 105.7148 93.4212) (size 0.8) (drill 0.4) (layers F.Cu B.Cu) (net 7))
 (segment (start 105.7148 98.5928) (end 105.7148 93.4212) (width 0.25) (layer F.Cu) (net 7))
 (segment (start 106.121 98.999) (end 105.7148 98.5928) (width 0.25) (layer F.Cu) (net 7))
 (segment (start 106.346 98.999) (end 106.121 98.999) (width 0.25) (layer F.Cu) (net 7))
 (segment (start 120.3452 93.4212) (end 120.396 93.472) (width 0.25) (layer B.Cu) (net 7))
 (segment (start 105.7148 93.4212) (end 120.3452 93.4212) (width 0.25) (layer B.Cu) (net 7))
 (segment (start 116.7384 88.2116) (end 116.492 88.458) (width 0.25) (layer F.Cu) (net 19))
 (segment (start 116.7384 86.36) (end 116.7384 88.2116) (width 0.25) (layer F.Cu) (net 19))
 (segment (start 113.792 90.358) (end 113.792 89.408) (width 0.5) (layer F.Cu) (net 3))
 (segment (start 107.121 100.899) (end 108.1345 99.8855) (width 0.25) (layer F.Cu) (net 3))
 (segment (start 106.346 100.899) (end 107.121 100.899) (width 0.25) (layer F.Cu) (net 3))
 (segment (start 110.7308 98.3874) (end 111.4933 97.6249) (width 0.25) (layer F.Cu) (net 3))
 (segment (start 109.569502 99.8855) (end 110.7308 98.724202) (width 0.25) (layer F.Cu) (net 3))
 (segment (start 110.7308 98.724202) (end 110.7308 98.3874) (width 0.25) (layer F.Cu) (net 3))
 (segment (start 108.1345 99.8855) (end 109.569502 99.8855) (width 0.25) (layer F.Cu) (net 3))
 (segment (start 111.4933 95.9499) (end 111.4933 97.6249) (width 0.25) (layer F.Cu) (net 3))
 (segment (start 113.042 90.358) (end 111.4933 91.9067) (width 0.5) (layer F.Cu) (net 3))
 (segment (start 111.4933 91.9067) (end 111.4933 95.9499) (width 0.5) (layer F.Cu) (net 3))
 (segment (start 113.792 90.358) (end 113.042 90.358) (width 0.5) (layer F.Cu) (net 3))
 (segment (start 109.956 81.538) (end 109.956 82.038) (width 0.25) (layer F.Cu) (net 17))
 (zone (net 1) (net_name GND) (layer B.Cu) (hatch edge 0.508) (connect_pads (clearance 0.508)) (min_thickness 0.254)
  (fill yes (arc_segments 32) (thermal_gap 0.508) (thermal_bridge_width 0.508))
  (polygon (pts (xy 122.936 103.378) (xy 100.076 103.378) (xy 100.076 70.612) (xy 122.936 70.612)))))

